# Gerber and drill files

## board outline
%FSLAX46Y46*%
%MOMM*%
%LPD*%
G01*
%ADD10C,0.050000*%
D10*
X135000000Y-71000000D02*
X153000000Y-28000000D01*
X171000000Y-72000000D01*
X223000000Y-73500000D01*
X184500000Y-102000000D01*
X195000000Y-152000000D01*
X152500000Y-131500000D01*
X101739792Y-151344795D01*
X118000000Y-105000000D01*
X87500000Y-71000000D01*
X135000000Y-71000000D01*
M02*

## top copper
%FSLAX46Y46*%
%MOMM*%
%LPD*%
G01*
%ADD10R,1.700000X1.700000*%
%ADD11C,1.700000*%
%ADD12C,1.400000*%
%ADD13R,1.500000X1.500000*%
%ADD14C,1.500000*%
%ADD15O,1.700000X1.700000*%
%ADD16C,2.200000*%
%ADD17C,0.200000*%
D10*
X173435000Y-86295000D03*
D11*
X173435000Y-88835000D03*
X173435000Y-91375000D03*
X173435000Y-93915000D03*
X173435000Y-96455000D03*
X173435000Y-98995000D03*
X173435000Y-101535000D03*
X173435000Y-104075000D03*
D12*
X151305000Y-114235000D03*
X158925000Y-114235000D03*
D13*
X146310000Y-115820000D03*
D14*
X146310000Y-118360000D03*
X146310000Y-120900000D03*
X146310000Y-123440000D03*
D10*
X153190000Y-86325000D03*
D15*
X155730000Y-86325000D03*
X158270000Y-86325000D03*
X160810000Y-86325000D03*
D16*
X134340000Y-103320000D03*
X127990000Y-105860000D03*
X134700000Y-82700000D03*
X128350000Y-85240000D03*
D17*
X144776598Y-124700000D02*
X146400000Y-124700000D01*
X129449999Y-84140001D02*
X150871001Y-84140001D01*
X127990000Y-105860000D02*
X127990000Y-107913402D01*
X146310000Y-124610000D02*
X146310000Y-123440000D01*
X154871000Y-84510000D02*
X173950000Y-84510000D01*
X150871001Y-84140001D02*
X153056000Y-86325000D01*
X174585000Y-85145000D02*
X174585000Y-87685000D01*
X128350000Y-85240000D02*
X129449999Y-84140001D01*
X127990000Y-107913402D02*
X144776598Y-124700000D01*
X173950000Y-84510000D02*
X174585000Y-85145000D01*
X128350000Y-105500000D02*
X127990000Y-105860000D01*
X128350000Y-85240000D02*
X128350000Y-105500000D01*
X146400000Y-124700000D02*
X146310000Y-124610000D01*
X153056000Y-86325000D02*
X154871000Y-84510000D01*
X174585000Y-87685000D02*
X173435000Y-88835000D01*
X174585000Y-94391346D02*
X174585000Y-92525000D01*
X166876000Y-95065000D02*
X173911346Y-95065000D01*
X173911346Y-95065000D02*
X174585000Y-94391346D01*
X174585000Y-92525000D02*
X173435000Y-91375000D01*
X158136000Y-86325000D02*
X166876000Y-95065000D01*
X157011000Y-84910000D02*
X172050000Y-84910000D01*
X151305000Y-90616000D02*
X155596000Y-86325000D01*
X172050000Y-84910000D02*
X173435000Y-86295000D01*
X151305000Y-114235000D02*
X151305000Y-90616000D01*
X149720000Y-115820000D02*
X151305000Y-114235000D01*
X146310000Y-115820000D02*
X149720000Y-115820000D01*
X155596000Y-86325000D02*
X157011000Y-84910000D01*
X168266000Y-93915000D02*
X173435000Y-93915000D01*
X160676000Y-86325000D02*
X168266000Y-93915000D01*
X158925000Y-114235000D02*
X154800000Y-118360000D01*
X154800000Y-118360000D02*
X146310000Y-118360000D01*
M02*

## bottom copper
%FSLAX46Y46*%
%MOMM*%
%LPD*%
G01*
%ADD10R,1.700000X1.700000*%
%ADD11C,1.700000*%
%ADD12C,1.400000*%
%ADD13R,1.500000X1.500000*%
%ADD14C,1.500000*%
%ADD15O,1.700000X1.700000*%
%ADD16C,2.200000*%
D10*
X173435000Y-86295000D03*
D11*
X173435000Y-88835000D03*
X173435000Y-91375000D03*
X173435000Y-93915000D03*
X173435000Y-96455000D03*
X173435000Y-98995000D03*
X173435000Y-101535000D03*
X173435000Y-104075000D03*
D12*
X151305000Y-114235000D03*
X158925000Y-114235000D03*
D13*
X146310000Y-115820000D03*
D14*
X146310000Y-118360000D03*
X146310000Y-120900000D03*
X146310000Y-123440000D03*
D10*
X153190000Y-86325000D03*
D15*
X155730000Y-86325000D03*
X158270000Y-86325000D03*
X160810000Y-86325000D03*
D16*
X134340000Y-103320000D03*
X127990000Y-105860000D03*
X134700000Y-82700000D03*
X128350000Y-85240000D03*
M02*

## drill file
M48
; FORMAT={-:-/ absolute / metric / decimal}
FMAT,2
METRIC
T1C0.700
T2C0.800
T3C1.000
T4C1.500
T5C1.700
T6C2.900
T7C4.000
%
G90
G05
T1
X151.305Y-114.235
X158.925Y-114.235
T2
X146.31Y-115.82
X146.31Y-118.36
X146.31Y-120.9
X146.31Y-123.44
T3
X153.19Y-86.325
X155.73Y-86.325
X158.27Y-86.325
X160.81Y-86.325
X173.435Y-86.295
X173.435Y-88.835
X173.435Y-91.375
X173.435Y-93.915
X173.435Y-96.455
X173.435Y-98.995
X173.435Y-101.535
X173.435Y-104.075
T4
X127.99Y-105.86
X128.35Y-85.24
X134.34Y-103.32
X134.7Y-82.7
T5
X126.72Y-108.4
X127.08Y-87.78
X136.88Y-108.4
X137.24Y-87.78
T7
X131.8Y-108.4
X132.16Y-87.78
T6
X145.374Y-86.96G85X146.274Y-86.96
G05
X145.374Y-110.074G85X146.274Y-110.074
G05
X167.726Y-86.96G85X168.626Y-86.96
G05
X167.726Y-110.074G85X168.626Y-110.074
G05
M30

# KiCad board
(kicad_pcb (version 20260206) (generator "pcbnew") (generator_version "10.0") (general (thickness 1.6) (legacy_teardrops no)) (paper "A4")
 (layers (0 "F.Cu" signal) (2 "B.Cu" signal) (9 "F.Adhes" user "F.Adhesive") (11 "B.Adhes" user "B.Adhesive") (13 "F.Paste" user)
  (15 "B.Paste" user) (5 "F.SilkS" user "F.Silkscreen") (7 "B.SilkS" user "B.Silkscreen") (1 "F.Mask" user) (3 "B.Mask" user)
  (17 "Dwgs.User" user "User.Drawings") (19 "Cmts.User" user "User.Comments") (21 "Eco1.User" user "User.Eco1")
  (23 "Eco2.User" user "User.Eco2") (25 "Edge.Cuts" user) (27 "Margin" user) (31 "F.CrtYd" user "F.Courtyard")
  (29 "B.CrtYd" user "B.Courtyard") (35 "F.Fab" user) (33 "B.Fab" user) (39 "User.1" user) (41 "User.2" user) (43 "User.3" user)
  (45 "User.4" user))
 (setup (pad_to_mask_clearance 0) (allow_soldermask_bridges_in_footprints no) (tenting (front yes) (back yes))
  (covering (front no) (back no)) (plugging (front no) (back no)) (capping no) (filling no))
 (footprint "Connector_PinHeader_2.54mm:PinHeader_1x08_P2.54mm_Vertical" (layer "F.Cu") (at 173.435 86.295)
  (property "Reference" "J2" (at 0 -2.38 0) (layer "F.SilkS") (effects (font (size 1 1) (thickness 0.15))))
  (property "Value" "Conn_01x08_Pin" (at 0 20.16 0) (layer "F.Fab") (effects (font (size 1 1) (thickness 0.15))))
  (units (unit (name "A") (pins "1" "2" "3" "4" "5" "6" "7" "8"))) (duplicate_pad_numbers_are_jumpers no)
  (pad "1" thru_hole rect (at 0 0) (size 1.7 1.7) (drill 1) (layers "*.Cu" "*.Mask") (remove_unused_layers no) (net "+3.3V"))
  (pad "2" thru_hole circle (at 0 2.54) (size 1.7 1.7) (drill 1) (layers "*.Cu" "*.Mask") (remove_unused_layers no) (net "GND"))
  (pad "3" thru_hole circle (at 0 5.08) (size 1.7 1.7) (drill 1) (layers "*.Cu" "*.Mask") (remove_unused_layers no) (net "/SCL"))
  (pad "4" thru_hole circle (at 0 7.62) (size 1.7 1.7) (drill 1) (layers "*.Cu" "*.Mask") (remove_unused_layers no) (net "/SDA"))
  (pad "5" thru_hole circle (at 0 10.16) (size 1.7 1.7) (drill 1) (layers "*.Cu" "*.Mask") (remove_unused_layers no)
   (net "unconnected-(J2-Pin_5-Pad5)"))
  (pad "6" thru_hole circle (at 0 12.7) (size 1.7 1.7) (drill 1) (layers "*.Cu" "*.Mask") (remove_unused_layers no)
   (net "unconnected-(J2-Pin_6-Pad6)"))
  (pad "7" thru_hole circle (at 0 15.24) (size 1.7 1.7) (drill 1) (layers "*.Cu" "*.Mask") (remove_unused_layers no)
   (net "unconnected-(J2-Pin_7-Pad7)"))
  (pad "8" thru_hole circle (at 0 17.78) (size 1.7 1.7) (drill 1) (layers "*.Cu" "*.Mask") (remove_unused_layers no)
   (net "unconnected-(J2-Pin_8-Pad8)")))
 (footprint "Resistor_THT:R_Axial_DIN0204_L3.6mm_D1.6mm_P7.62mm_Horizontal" (layer "F.Cu") (at 151.305 114.235)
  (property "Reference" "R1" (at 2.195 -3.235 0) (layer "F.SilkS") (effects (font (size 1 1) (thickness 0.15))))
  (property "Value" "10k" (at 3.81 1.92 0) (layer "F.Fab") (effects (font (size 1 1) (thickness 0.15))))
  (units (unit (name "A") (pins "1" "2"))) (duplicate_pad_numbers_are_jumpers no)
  (pad "1" thru_hole circle (at 0 0) (size 1.4 1.4) (drill 0.7) (layers "*.Cu" "*.Mask") (remove_unused_layers no) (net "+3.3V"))
  (pad "2" thru_hole circle (at 7.62 0) (size 1.4 1.4) (drill 0.7) (layers "*.Cu" "*.Mask") (remove_unused_layers no) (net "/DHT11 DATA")))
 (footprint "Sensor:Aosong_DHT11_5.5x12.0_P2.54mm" (layer "F.Cu") (at 146.31 115.82)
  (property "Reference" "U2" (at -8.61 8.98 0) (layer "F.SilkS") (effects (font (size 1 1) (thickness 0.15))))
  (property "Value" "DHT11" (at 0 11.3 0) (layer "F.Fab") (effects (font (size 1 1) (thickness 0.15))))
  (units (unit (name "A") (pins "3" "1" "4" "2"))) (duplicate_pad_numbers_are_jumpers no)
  (pad "1" thru_hole rect (at 0 0) (size 1.5 1.5) (drill 0.8) (layers "*.Cu" "*.Mask") (remove_unused_layers no) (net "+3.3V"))
  (pad "2" thru_hole circle (at 0 2.54) (size 1.5 1.5) (drill 0.8) (layers "*.Cu" "*.Mask") (remove_unused_layers no) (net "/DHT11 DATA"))
  (pad "3" thru_hole circle (at 0 5.08) (size 1.5 1.5) (drill 0.8) (layers "*.Cu" "*.Mask") (remove_unused_layers no)
   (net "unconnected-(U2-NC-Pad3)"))
  (pad "4" thru_hole circle (at 0 7.62) (size 1.5 1.5) (drill 0.8) (layers "*.Cu" "*.Mask") (remove_unused_layers no) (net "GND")))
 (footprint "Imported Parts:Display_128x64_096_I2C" (layer "F.Cu") (at 157 86.325)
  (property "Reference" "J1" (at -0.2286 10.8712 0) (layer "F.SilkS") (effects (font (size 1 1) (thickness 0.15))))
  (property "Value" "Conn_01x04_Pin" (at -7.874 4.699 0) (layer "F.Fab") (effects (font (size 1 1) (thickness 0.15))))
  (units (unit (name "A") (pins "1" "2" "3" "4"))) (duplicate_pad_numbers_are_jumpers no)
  (pad "" np_thru_hole oval (at -11.176 0.635) (size 3.8 2.9) (drill oval 3.8 2.9) (layers "*.Cu" "*.Mask"))
  (pad "" np_thru_hole oval (at -11.176 23.749) (size 3.8 2.9) (drill oval 3.8 2.9) (layers "*.Cu" "*.Mask"))
  (pad "" np_thru_hole oval (at 11.176 0.635) (size 3.8 2.9) (drill oval 3.8 2.9) (layers "*.Cu" "*.Mask"))
  (pad "" np_thru_hole oval (at 11.176 23.749) (size 3.8 2.9) (drill oval 3.8 2.9) (layers "*.Cu" "*.Mask"))
  (pad "1" thru_hole rect (at -3.81 0 90) (size 1.7 1.7) (drill 1) (layers "*.Cu" "*.Mask") (remove_unused_layers no) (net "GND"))
  (pad "2" thru_hole oval (at -1.27 0 90) (size 1.7 1.7) (drill 1) (layers "*.Cu" "*.Mask") (remove_unused_layers no) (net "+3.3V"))
  (pad "3" thru_hole oval (at 1.27 0 90) (size 1.7 1.7) (drill 1) (layers "*.Cu" "*.Mask") (remove_unused_layers no) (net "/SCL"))
  (pad "4" thru_hole oval (at 3.81 0 90) (size 1.7 1.7) (drill 1) (layers "*.Cu" "*.Mask") (remove_unused_layers no) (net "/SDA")))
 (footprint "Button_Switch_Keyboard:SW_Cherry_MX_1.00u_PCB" (layer "F.Cu") (at 134.34 103.32)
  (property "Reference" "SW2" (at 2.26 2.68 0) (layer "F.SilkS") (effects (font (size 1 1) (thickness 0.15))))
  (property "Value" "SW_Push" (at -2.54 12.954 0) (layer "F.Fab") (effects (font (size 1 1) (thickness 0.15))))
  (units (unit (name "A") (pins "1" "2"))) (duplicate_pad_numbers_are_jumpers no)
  (pad "" np_thru_hole circle (at -7.62 5.08) (size 1.7 1.7) (drill 1.7) (layers "*.Cu" "*.Mask"))
  (pad "" np_thru_hole circle (at -2.54 5.08) (size 4 4) (drill 4) (layers "*.Cu" "*.Mask"))
  (pad "" np_thru_hole circle (at 2.54 5.08) (size 1.7 1.7) (drill 1.7) (layers "*.Cu" "*.Mask"))
  (pad "1" thru_hole circle (at 0 0) (size 2.2 2.2) (drill 1.5) (layers "*.Cu" "*.Mask") (remove_unused_layers no) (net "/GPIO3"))
  (pad "2" thru_hole circle (at -6.35 2.54) (size 2.2 2.2) (drill 1.5) (layers "*.Cu" "*.Mask") (remove_unused_layers no) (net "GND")))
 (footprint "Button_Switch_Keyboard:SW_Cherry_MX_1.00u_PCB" (layer "F.Cu") (at 134.7 82.7)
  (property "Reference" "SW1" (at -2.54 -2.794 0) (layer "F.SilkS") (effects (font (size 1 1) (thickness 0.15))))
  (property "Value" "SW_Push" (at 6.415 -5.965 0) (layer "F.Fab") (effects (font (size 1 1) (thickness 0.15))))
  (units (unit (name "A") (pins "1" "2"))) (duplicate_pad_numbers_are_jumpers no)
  (pad "" np_thru_hole circle (at -7.62 5.08) (size 1.7 1.7) (drill 1.7) (layers "*.Cu" "*.Mask"))
  (pad "" np_thru_hole circle (at -2.54 5.08) (size 4 4) (drill 4) (layers "*.Cu" "*.Mask"))
  (pad "" np_thru_hole circle (at 2.54 5.08) (size 1.7 1.7) (drill 1.7) (layers "*.Cu" "*.Mask"))
  (pad "1" thru_hole circle (at 0 0) (size 2.2 2.2) (drill 1.5) (layers "*.Cu" "*.Mask") (remove_unused_layers no) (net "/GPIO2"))
  (pad "2" thru_hole circle (at -6.35 2.54) (size 2.2 2.2) (drill 1.5) (layers "*.Cu" "*.Mask") (remove_unused_layers no) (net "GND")))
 (gr_poly
  (pts (xy 135 71) (xy 153 28) (xy 171 72) (xy 223 73.5) (xy 184.5 102) (xy 195 152) (xy 152.5 131.5) (xy 101.739792 151.344795)
   (xy 118 105) (xy 87.5 71))
  (stroke (width 0.05) (type solid)) (fill no) (layer "Edge.Cuts"))
 (segment (start 144.776598 124.7) (end 146.4 124.7) (width 0.2) (layer "F.Cu") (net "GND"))
 (segment (start 129.449999 84.140001) (end 150.871001 84.140001) (width 0.2) (layer "F.Cu") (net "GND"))
 (segment (start 127.99 105.86) (end 127.99 107.913402) (width 0.2) (layer "F.Cu") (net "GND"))
 (segment (start 146.31 124.61) (end 146.31 123.44) (width 0.2) (layer "F.Cu") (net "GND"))
 (segment (start 154.871 84.51) (end 173.95 84.51) (width 0.2) (layer "F.Cu") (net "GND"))
 (segment (start 150.871001 84.140001) (end 153.056 86.325) (width 0.2) (layer "F.Cu") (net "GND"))
 (segment (start 174.585 85.145) (end 174.585 87.685) (width 0.2) (layer "F.Cu") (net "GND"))
 (segment (start 128.35 85.24) (end 129.449999 84.140001) (width 0.2) (layer "F.Cu") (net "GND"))
 (segment (start 127.99 107.913402) (end 144.776598 124.7) (width 0.2) (layer "F.Cu") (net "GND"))
 (segment (start 173.95 84.51) (end 174.585 85.145) (width 0.2) (layer "F.Cu") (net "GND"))
 (segment (start 128.35 105.5) (end 127.99 105.86) (width 0.2) (layer "F.Cu") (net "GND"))
 (segment (start 128.35 85.24) (end 128.35 105.5) (width 0.2) (layer "F.Cu") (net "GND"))
 (segment (start 146.4 124.7) (end 146.31 124.61) (width 0.2) (layer "F.Cu") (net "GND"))
 (segment (start 153.056 86.325) (end 154.871 84.51) (width 0.2) (layer "F.Cu") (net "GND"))
 (segment (start 174.585 87.685) (end 173.435 88.835) (width 0.2) (layer "F.Cu") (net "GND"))
 (segment (start 174.585 94.391346) (end 174.585 92.525) (width 0.2) (layer "F.Cu") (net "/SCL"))
 (segment (start 166.876 95.065) (end 173.911346 95.065) (width 0.2) (layer "F.Cu") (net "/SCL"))
 (segment (start 173.911346 95.065) (end 174.585 94.391346) (width 0.2) (layer "F.Cu") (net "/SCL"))
 (segment (start 174.585 92.525) (end 173.435 91.375) (width 0.2) (layer "F.Cu") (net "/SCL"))
 (segment (start 158.136 86.325) (end 166.876 95.065) (width 0.2) (layer "F.Cu") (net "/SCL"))
 (segment (start 157.011 84.91) (end 172.05 84.91) (width 0.2) (layer "F.Cu") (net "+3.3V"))
 (segment (start 151.305 90.616) (end 155.596 86.325) (width 0.2) (layer "F.Cu") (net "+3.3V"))
 (segment (start 172.05 84.91) (end 173.435 86.295) (width 0.2) (layer "F.Cu") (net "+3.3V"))
 (segment (start 151.305 114.235) (end 151.305 90.616) (width 0.2) (layer "F.Cu") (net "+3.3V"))
 (segment (start 149.72 115.82) (end 151.305 114.235) (width 0.2) (layer "F.Cu") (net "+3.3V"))
 (segment (start 146.31 115.82) (end 149.72 115.82) (width 0.2) (layer "F.Cu") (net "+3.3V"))
 (segment (start 155.596 86.325) (end 157.011 84.91) (width 0.2) (layer "F.Cu") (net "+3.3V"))
 (segment (start 168.266 93.915) (end 173.435 93.915) (width 0.2) (layer "F.Cu") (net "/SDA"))
 (segment (start 160.676 86.325) (end 168.266 93.915) (width 0.2) (layer "F.Cu") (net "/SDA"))
 (segment (start 158.925 114.235) (end 154.8 118.36) (width 0.2) (layer "F.Cu") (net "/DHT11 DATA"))
 (segment (start 154.8 118.36) (end 146.31 118.36) (width 0.2) (layer "F.Cu") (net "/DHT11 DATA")))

